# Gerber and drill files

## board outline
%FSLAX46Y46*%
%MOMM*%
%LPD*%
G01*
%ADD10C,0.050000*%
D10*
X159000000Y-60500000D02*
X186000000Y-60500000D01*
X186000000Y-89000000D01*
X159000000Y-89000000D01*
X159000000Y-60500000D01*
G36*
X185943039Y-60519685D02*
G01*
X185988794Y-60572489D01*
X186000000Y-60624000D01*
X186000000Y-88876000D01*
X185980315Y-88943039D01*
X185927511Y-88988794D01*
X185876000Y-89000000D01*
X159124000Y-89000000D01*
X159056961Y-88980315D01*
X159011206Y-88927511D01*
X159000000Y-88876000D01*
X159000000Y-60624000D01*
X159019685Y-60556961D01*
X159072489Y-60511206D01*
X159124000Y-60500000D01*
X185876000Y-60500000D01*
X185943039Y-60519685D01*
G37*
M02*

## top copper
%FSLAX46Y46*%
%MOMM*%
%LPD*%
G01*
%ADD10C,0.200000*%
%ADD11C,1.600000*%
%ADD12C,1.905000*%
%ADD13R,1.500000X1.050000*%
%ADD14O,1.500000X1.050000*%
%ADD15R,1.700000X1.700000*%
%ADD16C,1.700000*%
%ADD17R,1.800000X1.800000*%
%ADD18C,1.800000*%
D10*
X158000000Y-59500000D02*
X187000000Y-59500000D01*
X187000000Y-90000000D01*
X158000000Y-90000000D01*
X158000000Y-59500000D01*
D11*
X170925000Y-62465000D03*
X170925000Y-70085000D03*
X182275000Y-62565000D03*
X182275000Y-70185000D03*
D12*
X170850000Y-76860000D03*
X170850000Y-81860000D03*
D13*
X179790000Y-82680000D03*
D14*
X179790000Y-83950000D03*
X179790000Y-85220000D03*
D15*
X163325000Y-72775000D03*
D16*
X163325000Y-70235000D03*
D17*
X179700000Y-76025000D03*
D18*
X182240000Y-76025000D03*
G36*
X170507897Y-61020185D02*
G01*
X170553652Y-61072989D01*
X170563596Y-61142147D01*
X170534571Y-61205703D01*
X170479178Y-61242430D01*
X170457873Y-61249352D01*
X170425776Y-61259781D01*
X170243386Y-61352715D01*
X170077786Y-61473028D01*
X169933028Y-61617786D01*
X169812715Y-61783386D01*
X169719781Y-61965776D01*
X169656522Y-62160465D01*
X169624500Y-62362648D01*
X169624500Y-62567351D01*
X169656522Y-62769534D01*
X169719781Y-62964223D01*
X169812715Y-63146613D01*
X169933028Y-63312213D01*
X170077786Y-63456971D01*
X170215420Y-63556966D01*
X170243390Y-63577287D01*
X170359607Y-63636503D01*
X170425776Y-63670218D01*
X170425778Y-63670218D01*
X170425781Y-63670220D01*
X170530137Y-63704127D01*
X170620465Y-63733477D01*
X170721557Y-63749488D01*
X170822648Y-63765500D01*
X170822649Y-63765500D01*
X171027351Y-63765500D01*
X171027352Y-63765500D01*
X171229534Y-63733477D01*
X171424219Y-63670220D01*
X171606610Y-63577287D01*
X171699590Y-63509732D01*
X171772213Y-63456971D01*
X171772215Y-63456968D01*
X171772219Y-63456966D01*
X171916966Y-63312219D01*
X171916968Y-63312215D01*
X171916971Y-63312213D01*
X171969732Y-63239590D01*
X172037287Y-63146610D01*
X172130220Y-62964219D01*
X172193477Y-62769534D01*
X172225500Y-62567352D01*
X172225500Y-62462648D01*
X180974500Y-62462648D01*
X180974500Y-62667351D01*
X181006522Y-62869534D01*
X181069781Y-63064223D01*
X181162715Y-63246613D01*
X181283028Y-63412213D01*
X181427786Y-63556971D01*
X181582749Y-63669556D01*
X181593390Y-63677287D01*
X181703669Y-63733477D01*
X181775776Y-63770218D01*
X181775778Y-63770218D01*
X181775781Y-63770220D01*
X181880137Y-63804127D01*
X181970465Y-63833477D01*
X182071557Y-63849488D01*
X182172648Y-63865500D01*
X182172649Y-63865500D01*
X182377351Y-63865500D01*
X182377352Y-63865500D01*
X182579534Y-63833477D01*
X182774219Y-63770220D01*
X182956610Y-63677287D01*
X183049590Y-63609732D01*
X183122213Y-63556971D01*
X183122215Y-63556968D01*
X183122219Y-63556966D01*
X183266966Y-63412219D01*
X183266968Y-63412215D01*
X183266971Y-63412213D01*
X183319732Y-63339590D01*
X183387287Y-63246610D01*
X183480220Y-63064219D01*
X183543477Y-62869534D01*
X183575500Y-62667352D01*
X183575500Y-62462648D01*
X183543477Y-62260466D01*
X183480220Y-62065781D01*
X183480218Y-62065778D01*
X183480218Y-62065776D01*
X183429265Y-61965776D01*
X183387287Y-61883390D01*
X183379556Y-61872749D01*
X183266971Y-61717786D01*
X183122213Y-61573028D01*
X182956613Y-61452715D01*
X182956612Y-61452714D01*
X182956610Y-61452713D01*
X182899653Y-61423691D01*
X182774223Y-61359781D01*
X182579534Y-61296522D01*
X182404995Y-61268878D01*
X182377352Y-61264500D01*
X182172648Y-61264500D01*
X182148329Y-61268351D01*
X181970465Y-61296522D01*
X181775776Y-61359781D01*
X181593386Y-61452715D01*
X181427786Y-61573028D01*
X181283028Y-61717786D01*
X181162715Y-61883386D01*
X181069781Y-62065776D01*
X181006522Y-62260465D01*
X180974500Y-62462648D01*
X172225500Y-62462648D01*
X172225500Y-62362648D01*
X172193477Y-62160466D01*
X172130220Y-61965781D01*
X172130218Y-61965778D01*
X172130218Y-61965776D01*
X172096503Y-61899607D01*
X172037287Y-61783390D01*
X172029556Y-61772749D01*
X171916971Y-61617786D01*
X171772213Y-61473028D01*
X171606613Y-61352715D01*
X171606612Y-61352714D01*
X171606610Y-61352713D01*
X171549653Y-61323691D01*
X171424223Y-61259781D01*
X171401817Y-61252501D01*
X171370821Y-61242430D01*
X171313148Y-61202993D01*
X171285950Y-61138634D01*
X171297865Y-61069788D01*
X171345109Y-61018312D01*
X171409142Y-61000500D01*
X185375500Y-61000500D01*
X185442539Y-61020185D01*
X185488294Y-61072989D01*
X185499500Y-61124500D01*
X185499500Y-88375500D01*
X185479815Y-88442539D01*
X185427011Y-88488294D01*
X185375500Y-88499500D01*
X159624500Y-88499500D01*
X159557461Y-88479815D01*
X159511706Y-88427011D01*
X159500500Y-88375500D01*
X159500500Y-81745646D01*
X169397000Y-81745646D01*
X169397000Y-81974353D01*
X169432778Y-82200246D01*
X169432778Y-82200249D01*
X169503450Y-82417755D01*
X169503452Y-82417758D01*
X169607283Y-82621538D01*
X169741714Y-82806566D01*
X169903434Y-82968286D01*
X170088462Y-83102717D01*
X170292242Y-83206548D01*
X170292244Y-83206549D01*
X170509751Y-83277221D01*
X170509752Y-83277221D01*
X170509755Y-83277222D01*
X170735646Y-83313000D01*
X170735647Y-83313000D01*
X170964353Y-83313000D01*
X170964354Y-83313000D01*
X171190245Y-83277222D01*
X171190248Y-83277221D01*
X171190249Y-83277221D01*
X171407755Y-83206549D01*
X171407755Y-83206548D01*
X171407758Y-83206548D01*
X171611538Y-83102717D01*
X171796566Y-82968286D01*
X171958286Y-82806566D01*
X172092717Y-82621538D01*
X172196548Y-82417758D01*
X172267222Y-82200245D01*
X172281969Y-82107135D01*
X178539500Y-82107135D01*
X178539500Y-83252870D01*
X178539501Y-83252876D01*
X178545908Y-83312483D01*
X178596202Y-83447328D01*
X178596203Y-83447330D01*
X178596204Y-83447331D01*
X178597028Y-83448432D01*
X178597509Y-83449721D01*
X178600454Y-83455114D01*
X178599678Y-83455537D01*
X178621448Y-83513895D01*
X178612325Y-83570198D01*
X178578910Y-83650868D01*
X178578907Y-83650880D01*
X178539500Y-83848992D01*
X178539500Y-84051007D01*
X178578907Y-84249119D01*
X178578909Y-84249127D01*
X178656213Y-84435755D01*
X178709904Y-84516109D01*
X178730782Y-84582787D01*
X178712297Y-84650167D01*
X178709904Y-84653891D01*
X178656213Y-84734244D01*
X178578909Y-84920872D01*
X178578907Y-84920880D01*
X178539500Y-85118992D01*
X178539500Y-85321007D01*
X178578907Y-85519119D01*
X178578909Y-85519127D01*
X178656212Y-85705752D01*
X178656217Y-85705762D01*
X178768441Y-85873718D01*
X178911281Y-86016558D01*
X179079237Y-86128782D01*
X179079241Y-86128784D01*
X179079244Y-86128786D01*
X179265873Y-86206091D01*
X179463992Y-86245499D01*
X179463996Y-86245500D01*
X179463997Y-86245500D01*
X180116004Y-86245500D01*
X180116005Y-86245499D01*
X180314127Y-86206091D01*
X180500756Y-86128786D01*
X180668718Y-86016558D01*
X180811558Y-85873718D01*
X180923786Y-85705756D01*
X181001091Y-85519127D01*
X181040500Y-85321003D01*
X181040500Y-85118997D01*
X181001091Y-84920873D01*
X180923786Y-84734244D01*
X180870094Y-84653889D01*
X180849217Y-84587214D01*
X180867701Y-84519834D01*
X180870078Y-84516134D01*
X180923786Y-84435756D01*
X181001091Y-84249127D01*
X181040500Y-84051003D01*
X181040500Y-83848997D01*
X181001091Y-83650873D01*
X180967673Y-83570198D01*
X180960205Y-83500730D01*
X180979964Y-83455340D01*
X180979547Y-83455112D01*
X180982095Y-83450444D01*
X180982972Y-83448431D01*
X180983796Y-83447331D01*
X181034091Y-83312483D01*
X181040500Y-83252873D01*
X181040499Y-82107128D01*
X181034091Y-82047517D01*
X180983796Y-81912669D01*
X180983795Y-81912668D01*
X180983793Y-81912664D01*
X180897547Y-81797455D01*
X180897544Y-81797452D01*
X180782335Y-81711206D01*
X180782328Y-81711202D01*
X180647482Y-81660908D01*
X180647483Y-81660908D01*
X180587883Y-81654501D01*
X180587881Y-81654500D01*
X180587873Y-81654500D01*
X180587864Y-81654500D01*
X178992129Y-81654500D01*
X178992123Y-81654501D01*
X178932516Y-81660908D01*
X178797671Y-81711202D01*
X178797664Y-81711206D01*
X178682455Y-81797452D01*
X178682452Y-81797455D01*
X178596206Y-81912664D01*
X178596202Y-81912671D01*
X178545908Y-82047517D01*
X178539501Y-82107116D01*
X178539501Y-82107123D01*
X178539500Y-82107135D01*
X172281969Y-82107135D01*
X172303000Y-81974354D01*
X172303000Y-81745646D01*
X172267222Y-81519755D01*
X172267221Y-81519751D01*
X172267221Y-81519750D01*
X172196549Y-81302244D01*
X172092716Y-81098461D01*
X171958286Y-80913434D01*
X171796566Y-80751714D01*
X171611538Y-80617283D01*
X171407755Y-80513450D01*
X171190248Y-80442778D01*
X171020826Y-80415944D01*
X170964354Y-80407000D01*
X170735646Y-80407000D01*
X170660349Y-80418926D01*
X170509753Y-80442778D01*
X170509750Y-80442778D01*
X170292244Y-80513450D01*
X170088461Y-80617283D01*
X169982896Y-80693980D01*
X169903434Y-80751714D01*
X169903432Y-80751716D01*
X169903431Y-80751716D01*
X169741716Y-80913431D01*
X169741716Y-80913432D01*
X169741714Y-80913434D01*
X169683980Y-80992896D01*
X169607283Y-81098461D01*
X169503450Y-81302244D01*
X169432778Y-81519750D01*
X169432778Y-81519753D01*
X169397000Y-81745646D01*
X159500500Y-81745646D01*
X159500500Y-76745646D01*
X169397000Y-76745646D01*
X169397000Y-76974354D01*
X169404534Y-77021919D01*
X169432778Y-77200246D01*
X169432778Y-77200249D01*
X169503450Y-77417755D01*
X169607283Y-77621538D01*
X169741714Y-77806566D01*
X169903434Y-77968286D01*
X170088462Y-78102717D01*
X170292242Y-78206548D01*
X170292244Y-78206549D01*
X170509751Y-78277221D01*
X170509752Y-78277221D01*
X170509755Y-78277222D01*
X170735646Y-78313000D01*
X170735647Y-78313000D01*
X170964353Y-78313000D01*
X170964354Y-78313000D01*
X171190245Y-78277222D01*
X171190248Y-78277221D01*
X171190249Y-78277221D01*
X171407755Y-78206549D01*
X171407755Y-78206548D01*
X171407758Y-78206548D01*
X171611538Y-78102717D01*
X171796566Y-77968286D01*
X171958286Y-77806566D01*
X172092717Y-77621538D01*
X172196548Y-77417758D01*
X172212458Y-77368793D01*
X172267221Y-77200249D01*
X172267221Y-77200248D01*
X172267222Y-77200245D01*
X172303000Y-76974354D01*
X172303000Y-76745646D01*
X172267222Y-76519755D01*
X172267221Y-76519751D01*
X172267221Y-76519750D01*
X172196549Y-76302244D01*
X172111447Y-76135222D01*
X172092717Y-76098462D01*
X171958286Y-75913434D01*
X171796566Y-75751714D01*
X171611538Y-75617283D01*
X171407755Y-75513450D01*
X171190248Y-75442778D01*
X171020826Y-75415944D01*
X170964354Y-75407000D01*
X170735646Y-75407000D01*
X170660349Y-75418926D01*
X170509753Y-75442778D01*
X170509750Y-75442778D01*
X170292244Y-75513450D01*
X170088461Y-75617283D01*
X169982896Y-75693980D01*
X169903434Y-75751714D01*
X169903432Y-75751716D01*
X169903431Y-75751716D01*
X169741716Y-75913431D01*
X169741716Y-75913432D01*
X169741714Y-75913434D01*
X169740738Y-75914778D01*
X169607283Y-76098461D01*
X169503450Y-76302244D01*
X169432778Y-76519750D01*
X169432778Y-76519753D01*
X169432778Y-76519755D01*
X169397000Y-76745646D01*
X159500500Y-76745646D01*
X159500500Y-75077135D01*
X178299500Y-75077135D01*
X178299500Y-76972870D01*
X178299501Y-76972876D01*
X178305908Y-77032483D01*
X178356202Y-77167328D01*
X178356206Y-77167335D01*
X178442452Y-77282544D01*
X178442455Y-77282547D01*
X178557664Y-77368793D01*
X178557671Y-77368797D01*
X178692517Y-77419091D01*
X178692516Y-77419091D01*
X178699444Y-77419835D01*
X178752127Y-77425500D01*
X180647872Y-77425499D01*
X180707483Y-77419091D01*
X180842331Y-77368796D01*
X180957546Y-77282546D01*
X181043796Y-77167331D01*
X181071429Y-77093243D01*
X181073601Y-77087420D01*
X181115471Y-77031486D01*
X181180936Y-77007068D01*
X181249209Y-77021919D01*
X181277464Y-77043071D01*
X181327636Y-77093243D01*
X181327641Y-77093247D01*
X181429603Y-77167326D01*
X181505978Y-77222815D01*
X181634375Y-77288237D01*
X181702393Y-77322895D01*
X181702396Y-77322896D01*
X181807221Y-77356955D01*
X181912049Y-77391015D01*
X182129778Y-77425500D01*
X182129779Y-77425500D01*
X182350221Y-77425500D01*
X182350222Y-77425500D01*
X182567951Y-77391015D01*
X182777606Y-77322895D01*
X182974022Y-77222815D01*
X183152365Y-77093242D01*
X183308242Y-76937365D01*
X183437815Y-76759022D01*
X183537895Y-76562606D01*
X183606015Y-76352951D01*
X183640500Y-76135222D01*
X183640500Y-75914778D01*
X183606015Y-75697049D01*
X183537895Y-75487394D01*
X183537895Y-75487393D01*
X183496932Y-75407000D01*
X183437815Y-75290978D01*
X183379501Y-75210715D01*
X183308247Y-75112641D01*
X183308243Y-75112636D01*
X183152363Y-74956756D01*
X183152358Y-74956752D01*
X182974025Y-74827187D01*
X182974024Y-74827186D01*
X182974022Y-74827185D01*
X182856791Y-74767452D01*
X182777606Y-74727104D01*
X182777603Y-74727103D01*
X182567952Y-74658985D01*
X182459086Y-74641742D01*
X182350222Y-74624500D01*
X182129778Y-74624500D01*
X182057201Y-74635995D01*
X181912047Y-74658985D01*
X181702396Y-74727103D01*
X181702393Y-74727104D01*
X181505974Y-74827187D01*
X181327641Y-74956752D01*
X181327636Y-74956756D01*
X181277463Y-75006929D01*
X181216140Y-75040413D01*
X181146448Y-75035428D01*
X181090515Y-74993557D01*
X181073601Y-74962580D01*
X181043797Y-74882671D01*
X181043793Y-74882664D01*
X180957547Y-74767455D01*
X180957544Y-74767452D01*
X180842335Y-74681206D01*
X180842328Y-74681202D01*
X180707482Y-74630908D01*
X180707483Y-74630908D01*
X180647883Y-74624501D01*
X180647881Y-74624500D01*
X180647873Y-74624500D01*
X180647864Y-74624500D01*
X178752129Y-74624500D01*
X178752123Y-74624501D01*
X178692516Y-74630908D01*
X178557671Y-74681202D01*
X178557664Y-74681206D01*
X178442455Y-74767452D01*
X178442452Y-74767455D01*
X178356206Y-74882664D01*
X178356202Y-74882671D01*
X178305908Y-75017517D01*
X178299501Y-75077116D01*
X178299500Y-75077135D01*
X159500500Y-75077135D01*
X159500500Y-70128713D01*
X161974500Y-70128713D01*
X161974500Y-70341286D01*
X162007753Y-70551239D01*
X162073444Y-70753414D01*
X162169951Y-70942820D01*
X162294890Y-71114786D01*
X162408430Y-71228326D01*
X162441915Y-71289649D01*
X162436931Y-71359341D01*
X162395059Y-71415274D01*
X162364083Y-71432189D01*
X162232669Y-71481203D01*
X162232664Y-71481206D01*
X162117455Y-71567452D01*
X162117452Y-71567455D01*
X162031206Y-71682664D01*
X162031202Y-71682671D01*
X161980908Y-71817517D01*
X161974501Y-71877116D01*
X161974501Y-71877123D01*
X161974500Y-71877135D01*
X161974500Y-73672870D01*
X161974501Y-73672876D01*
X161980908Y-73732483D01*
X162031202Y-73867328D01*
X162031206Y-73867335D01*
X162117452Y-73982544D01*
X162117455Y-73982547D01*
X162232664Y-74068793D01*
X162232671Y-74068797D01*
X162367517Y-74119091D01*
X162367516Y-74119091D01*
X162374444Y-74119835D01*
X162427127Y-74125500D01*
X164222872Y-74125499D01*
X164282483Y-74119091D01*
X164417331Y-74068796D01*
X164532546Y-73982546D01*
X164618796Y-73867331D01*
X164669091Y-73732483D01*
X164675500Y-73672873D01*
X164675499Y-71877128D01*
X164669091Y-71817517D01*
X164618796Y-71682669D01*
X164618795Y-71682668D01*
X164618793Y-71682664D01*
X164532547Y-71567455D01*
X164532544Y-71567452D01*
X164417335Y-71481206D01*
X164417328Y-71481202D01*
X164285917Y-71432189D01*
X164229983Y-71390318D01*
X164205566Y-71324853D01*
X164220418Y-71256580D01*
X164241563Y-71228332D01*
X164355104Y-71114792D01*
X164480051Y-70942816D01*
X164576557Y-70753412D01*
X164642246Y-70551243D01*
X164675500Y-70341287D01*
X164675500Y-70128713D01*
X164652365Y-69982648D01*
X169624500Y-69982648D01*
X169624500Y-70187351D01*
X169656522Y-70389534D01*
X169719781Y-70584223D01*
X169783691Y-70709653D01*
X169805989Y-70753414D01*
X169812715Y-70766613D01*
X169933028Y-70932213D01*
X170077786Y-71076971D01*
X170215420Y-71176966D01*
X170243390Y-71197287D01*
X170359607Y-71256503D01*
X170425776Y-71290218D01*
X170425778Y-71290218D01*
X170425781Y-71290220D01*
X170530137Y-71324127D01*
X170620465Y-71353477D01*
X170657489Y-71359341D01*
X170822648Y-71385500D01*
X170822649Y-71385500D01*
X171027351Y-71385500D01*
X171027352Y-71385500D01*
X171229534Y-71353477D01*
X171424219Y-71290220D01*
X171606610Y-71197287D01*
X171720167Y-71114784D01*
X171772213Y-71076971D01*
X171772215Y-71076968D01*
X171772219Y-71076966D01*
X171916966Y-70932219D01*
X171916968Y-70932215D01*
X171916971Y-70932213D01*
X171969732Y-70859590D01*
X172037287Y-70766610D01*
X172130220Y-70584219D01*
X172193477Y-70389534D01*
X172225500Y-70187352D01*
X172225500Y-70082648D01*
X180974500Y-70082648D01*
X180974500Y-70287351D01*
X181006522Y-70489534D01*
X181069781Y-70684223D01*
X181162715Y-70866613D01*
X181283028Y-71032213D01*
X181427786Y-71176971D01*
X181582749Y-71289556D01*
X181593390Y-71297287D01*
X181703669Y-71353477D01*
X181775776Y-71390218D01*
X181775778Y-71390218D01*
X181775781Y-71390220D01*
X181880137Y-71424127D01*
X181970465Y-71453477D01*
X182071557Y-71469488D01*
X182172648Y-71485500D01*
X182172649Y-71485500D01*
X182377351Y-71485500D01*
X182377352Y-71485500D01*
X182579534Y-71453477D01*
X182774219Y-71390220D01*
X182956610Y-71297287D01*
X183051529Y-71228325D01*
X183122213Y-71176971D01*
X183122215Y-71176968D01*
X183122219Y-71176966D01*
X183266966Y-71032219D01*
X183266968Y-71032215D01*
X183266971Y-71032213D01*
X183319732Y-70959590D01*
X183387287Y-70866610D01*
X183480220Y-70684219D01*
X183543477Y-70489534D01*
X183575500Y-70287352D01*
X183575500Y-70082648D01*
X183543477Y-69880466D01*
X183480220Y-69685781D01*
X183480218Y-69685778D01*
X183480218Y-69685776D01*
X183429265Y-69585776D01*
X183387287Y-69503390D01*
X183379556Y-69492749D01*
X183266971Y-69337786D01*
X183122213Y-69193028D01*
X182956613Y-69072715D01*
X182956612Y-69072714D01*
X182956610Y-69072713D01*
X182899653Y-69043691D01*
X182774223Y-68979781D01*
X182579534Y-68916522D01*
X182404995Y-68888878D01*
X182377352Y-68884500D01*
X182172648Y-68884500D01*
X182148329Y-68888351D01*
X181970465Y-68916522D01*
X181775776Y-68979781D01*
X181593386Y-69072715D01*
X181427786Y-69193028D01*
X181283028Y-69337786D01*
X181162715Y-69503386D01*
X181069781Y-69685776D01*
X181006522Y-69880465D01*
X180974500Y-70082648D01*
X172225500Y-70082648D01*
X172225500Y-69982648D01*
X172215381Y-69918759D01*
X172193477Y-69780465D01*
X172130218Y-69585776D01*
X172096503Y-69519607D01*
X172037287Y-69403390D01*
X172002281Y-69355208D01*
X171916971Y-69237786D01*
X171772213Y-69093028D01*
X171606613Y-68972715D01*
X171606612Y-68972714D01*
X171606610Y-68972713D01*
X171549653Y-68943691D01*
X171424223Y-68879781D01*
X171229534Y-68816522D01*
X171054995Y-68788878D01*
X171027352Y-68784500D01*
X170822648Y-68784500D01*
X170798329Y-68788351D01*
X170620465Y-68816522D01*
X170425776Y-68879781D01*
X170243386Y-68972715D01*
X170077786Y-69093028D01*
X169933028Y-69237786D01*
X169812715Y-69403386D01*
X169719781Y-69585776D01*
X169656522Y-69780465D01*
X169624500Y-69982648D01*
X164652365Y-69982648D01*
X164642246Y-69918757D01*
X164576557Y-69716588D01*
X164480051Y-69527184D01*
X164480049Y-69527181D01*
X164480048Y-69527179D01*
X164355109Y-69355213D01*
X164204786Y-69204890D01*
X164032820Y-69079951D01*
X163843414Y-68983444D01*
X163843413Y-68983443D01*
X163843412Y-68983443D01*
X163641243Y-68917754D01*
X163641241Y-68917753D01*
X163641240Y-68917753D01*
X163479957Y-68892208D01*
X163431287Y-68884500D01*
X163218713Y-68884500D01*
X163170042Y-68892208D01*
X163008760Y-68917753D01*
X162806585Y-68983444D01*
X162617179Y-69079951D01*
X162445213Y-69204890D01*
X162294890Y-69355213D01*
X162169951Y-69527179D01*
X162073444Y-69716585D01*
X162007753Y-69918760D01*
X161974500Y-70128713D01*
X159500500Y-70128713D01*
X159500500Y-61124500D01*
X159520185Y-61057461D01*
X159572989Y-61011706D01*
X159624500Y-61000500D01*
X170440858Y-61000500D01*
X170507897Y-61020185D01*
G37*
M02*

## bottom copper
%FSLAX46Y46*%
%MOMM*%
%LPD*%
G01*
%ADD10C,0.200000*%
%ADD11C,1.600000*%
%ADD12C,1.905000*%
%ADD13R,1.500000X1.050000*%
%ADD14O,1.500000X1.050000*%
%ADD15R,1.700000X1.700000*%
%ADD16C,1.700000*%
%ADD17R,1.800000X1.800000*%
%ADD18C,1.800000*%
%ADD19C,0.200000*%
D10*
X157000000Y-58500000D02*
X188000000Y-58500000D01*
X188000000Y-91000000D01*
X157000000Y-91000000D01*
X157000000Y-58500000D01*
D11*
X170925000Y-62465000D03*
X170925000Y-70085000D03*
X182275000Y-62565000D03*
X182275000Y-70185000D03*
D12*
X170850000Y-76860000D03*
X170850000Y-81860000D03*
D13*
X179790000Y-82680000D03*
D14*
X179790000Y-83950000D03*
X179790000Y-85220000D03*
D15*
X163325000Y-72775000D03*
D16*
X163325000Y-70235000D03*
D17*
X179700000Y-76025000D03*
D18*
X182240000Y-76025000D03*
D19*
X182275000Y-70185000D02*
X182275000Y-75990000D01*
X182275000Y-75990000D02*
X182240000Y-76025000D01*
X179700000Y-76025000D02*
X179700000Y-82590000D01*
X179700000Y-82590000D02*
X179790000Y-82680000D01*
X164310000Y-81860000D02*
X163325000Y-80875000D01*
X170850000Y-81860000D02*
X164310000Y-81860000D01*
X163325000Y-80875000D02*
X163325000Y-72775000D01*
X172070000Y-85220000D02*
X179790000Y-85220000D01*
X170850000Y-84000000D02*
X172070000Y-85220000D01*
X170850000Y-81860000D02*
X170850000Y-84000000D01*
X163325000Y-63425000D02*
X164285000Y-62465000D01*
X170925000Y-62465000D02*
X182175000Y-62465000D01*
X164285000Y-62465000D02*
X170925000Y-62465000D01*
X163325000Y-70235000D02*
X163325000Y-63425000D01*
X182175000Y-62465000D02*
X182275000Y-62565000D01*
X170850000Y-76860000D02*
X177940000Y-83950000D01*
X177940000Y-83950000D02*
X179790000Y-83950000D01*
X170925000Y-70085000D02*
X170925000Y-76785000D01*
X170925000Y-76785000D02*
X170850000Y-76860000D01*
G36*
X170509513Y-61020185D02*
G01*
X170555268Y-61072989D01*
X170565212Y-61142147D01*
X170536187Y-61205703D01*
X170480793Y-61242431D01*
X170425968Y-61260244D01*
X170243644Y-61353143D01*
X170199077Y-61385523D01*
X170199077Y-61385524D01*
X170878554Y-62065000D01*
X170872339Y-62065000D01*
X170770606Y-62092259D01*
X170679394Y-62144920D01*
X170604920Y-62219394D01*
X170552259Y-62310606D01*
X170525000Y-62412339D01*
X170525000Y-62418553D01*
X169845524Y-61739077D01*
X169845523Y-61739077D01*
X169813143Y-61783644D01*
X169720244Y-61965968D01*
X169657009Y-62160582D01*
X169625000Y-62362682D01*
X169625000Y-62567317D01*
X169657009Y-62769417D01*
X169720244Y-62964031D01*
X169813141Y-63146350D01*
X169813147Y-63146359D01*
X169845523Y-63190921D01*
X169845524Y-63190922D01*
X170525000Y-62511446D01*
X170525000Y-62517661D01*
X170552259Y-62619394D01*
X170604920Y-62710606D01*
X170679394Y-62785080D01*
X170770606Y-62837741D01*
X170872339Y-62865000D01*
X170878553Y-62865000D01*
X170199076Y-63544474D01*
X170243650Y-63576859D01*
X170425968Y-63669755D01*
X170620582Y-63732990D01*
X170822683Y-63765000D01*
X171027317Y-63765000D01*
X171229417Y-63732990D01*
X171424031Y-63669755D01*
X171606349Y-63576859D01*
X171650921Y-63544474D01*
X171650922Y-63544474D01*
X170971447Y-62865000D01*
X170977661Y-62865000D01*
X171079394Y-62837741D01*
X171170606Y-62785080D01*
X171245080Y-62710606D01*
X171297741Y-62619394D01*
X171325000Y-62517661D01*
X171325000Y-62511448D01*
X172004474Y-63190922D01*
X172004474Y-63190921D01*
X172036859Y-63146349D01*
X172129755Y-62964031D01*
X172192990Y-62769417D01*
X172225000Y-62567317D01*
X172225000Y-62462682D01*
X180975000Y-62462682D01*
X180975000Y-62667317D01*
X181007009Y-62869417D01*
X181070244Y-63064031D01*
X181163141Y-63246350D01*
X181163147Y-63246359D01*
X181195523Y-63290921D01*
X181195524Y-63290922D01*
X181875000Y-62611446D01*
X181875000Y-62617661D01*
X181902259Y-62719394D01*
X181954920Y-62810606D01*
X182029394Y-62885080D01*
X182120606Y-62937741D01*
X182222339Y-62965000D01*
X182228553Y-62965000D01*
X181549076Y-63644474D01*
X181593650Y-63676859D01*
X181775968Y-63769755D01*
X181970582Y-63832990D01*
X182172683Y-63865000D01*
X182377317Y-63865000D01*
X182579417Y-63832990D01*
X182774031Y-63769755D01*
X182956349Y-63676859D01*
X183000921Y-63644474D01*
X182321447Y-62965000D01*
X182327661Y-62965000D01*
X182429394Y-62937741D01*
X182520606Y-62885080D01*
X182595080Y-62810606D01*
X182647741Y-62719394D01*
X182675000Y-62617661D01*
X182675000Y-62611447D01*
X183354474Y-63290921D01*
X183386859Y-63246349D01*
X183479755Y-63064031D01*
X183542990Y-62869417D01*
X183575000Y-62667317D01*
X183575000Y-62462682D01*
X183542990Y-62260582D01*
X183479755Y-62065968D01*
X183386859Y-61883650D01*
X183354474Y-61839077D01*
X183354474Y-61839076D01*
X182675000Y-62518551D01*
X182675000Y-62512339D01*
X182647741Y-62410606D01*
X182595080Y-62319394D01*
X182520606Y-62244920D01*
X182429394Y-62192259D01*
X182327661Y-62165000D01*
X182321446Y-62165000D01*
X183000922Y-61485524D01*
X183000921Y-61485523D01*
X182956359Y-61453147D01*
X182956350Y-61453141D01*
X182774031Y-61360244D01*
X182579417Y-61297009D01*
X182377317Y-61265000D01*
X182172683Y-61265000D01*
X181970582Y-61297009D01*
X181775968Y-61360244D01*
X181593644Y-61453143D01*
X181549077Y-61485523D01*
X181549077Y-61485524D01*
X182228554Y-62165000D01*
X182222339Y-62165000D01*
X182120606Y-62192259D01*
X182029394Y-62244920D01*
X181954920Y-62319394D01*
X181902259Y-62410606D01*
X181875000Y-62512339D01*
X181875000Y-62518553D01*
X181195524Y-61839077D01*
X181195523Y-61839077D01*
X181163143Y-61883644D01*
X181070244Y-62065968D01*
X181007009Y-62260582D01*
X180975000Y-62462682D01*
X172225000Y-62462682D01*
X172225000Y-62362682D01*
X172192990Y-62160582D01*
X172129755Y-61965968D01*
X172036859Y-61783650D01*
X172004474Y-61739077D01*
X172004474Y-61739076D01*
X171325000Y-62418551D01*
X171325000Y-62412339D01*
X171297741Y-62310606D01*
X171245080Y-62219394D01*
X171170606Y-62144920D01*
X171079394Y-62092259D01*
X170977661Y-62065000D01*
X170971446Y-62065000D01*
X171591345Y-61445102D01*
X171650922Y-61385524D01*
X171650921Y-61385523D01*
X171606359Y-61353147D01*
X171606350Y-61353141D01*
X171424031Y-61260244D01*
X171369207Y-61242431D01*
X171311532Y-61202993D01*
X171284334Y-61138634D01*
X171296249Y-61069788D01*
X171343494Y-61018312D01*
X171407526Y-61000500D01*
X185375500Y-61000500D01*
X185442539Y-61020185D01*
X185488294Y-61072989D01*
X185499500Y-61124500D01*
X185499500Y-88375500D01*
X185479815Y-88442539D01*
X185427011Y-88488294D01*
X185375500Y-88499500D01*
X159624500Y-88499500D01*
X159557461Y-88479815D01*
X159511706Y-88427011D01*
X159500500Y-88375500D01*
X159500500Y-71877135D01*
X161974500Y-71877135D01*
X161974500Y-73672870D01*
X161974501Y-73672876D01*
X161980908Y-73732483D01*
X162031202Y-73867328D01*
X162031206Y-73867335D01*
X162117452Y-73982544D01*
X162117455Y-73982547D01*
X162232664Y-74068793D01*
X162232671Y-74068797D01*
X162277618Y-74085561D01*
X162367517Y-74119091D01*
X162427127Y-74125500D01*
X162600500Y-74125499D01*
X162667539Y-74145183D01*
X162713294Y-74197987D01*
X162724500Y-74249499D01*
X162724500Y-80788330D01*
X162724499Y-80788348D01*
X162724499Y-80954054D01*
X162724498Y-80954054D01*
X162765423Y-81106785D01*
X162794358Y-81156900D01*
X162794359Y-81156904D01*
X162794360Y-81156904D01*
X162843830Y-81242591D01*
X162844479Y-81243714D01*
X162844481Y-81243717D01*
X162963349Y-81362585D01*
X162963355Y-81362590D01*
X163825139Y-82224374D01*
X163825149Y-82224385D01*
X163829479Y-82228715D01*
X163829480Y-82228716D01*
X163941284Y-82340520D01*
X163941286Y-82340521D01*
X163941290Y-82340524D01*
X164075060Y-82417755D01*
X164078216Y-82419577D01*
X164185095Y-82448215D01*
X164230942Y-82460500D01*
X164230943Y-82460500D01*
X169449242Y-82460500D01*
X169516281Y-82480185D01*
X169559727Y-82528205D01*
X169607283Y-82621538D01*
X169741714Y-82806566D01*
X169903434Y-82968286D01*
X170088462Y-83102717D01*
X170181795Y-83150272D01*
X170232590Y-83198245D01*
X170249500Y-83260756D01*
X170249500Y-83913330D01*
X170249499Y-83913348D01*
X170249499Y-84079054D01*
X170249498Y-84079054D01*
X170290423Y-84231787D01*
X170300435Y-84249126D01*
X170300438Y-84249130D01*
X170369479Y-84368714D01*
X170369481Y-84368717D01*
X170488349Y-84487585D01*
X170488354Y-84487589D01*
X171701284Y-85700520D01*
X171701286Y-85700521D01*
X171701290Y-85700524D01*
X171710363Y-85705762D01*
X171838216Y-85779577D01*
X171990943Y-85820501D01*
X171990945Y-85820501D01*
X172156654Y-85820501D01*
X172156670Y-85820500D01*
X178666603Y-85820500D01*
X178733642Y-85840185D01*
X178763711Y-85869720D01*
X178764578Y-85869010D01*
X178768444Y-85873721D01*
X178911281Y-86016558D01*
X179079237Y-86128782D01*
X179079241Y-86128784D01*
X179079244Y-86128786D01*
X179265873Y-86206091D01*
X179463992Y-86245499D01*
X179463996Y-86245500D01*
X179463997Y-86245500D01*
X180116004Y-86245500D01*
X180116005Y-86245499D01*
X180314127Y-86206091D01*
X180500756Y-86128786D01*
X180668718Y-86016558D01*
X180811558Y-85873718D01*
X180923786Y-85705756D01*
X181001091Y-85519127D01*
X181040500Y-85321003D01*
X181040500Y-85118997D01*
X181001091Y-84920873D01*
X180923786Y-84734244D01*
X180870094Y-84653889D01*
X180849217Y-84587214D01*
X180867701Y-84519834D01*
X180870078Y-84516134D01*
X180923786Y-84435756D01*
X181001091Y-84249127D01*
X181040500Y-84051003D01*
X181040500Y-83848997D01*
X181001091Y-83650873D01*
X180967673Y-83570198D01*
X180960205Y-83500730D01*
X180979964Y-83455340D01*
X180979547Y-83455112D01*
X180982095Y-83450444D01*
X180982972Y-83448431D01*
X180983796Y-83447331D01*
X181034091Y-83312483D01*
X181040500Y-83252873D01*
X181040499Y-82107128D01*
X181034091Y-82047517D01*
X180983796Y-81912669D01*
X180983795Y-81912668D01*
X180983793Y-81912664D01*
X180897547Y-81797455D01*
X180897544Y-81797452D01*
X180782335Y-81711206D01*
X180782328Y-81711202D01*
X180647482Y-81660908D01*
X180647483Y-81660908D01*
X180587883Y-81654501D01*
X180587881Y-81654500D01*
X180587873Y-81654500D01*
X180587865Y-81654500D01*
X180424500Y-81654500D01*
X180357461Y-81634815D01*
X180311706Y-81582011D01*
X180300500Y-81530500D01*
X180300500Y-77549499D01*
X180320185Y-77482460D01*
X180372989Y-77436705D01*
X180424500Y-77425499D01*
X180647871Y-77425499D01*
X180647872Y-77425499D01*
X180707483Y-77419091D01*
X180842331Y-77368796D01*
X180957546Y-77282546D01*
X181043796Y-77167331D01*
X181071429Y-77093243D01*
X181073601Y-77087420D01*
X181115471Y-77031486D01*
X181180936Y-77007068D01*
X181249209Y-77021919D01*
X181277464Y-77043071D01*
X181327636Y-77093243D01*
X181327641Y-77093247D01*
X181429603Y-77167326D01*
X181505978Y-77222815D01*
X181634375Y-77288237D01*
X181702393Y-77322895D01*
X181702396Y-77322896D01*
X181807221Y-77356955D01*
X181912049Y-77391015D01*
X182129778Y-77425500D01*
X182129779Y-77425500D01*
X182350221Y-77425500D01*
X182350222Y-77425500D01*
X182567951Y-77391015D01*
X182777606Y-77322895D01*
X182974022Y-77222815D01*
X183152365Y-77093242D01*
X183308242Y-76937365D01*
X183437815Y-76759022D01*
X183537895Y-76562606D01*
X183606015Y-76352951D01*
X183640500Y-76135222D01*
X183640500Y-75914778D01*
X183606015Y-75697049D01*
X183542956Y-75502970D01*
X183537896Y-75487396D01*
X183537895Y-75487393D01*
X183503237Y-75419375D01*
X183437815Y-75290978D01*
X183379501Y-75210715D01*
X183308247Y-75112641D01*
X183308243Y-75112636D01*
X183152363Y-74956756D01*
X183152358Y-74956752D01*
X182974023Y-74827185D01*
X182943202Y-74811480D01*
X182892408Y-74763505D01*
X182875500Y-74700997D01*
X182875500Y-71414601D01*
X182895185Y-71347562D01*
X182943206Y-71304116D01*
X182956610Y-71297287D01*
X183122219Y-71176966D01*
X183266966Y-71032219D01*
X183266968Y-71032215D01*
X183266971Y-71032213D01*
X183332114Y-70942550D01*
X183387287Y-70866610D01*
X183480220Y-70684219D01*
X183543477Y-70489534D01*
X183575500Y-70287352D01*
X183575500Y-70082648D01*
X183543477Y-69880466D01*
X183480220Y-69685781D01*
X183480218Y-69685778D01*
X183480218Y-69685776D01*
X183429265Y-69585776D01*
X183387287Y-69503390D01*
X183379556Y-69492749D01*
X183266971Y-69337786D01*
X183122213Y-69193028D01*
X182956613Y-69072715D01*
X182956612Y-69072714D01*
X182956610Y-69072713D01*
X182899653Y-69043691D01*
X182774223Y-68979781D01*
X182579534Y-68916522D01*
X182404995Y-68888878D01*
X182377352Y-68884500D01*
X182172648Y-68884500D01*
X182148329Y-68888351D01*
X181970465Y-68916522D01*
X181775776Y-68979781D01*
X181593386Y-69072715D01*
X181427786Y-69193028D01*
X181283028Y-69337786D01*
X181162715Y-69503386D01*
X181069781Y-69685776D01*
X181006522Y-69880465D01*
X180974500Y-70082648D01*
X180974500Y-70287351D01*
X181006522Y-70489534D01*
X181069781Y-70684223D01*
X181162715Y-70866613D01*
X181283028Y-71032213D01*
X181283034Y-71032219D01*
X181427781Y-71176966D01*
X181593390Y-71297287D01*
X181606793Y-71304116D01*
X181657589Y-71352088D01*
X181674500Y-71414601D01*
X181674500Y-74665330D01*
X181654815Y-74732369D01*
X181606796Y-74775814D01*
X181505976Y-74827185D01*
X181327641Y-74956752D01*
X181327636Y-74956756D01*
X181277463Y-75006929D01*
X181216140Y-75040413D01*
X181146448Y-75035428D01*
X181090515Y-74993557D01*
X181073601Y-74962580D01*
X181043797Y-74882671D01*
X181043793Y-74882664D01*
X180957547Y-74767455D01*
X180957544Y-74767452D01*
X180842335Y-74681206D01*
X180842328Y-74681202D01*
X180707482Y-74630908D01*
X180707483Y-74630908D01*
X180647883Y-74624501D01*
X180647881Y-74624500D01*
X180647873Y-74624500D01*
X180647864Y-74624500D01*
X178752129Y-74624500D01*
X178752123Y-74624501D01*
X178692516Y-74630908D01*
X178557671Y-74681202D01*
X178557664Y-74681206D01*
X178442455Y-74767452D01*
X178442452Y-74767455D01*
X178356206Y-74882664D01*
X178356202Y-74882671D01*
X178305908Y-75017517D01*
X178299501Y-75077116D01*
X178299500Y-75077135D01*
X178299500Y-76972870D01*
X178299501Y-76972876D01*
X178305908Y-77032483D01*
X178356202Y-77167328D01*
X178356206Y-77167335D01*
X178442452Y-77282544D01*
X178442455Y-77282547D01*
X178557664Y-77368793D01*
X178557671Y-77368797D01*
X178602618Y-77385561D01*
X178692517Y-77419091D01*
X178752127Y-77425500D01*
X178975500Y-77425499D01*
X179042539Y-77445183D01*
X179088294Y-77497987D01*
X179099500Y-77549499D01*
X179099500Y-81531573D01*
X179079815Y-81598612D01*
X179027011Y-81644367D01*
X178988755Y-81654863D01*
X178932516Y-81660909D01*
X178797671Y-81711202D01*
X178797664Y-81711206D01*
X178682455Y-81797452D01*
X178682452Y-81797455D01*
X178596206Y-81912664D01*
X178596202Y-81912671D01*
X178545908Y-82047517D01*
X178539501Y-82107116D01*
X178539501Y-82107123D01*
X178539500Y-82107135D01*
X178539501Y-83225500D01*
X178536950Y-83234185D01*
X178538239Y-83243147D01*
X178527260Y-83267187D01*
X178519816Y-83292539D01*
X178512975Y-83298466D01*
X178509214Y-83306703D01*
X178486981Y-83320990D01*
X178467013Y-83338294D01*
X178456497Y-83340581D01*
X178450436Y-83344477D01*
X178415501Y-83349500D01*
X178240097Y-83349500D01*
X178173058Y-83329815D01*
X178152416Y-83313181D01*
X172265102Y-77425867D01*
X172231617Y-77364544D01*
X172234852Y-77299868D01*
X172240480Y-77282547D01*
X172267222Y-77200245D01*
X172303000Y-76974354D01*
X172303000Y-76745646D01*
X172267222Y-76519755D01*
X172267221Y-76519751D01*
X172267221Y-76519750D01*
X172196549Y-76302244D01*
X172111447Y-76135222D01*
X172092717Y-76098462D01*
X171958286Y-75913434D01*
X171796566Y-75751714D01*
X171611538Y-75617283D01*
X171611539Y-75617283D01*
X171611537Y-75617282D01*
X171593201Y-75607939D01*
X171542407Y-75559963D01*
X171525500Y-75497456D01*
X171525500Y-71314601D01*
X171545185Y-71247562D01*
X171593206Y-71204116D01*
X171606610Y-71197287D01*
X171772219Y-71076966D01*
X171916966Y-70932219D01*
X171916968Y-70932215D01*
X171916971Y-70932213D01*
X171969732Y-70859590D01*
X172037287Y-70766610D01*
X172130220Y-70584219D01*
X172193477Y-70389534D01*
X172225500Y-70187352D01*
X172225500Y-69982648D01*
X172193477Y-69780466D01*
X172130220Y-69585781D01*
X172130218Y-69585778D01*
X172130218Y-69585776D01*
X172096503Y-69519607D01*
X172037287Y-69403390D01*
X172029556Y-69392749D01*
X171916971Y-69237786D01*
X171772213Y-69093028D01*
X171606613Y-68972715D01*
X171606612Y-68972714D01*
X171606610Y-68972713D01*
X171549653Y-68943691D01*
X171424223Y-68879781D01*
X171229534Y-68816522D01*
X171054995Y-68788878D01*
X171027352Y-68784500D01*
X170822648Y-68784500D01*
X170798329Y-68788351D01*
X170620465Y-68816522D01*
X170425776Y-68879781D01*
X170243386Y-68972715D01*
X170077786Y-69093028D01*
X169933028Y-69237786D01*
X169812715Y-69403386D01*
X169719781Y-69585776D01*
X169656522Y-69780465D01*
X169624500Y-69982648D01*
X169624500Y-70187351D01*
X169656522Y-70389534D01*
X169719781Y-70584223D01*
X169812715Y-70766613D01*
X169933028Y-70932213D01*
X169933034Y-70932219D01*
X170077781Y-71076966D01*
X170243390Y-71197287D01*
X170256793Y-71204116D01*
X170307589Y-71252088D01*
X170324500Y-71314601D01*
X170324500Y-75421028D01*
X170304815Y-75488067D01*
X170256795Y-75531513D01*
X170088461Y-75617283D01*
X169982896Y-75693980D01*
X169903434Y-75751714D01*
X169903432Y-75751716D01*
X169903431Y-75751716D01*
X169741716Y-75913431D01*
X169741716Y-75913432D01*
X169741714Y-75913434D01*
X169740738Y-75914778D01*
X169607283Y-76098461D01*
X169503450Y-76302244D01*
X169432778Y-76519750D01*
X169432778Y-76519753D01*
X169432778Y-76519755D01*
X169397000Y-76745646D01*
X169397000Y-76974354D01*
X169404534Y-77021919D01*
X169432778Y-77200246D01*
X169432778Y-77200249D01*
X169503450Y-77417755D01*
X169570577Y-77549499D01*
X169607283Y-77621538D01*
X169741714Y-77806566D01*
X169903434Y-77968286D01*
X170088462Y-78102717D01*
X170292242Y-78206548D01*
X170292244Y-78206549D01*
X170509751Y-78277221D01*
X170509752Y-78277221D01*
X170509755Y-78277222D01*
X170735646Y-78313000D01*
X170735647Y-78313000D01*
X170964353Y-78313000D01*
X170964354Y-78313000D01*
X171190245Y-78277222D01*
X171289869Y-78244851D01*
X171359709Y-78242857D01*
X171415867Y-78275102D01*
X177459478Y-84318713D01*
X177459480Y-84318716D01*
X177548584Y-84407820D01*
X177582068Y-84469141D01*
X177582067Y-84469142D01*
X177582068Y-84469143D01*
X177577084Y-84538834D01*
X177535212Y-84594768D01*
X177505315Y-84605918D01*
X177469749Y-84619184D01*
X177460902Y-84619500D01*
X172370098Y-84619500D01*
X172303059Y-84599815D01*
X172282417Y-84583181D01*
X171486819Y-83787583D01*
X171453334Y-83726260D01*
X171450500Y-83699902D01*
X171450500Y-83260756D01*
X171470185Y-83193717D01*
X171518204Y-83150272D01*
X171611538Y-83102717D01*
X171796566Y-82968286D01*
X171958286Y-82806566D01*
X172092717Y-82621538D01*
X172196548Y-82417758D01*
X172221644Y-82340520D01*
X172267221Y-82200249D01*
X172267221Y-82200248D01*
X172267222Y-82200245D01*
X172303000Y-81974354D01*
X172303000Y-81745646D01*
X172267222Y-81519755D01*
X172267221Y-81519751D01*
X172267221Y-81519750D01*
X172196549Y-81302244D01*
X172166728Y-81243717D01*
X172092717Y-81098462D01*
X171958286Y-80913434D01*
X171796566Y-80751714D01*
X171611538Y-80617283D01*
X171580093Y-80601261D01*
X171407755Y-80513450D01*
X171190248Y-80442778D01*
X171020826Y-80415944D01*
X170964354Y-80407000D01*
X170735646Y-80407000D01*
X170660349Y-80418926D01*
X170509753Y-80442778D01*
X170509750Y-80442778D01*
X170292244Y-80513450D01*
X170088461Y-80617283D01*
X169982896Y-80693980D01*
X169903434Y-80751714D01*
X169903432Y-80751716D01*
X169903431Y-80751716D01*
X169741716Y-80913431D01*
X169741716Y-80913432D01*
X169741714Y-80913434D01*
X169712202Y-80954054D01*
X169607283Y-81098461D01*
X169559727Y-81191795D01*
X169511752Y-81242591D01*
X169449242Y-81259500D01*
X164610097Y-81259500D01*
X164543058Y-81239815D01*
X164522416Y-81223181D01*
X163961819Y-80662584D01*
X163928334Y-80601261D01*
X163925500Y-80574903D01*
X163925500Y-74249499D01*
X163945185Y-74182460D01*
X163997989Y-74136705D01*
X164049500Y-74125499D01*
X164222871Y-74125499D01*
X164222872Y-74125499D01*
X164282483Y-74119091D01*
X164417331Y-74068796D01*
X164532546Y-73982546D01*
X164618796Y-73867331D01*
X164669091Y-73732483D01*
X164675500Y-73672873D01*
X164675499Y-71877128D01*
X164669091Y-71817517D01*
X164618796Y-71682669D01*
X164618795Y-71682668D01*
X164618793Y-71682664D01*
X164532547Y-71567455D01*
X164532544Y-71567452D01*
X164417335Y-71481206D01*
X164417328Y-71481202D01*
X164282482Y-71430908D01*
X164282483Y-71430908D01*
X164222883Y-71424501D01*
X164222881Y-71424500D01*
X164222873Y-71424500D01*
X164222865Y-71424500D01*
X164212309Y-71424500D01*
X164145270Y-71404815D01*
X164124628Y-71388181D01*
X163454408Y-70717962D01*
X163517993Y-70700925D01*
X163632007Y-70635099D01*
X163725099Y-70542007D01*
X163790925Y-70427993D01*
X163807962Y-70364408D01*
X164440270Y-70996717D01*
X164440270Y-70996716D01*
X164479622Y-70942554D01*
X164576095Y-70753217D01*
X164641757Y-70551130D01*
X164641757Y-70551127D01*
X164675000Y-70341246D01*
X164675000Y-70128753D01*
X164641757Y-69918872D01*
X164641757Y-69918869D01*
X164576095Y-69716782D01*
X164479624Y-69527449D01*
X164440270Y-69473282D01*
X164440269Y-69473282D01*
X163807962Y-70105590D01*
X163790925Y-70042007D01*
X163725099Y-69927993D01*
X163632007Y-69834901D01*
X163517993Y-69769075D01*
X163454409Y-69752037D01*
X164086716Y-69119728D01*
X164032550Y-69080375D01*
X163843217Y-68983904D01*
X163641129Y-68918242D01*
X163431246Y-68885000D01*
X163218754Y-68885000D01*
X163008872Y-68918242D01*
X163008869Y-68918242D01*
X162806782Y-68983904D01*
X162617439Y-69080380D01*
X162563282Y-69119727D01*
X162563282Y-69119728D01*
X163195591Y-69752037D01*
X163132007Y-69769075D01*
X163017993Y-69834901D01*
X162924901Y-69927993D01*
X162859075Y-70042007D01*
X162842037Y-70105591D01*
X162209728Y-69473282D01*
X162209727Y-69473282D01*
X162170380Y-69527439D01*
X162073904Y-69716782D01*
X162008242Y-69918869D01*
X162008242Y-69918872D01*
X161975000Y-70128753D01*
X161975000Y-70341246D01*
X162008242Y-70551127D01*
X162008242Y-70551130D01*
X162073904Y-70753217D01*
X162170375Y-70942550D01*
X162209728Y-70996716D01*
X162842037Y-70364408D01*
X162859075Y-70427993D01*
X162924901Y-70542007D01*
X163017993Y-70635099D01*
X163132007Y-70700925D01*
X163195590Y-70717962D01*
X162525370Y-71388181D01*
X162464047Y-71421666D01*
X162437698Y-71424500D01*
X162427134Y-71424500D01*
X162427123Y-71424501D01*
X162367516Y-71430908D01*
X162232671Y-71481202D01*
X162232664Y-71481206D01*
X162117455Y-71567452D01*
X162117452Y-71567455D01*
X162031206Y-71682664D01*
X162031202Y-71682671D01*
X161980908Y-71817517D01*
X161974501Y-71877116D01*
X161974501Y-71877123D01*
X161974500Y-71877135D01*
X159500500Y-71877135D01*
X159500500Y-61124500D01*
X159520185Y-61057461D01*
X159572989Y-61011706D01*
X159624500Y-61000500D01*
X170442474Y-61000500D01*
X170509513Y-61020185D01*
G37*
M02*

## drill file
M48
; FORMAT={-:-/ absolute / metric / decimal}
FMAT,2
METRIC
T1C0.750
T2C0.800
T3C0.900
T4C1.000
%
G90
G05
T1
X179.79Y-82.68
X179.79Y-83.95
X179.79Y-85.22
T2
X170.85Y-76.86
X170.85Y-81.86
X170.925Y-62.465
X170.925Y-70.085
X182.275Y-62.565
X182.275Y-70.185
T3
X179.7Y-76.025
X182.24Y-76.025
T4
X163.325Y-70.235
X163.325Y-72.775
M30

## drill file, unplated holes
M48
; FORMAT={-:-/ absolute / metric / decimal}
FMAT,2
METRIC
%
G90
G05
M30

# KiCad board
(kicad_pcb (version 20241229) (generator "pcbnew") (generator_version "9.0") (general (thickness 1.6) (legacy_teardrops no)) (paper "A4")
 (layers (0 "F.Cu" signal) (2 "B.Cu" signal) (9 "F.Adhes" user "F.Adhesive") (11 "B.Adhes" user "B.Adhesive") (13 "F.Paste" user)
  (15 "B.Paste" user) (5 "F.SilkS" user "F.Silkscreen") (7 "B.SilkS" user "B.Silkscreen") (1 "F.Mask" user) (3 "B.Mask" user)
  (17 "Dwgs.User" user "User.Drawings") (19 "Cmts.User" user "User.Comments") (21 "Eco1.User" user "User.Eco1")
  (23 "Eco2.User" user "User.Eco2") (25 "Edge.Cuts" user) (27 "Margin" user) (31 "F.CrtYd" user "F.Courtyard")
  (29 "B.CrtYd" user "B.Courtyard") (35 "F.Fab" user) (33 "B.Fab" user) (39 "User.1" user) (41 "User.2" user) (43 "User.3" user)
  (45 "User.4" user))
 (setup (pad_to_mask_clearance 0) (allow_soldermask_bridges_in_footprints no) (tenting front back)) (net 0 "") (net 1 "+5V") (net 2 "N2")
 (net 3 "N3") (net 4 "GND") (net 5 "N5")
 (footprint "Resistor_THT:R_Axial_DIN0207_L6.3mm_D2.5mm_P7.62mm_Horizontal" (layer "F.Cu") (at 170.925 62.465 -90)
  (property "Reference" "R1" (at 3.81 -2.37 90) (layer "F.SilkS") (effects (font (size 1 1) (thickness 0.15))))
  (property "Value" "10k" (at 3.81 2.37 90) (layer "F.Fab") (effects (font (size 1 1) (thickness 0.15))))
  (pad "1" thru_hole circle (at 0 0 270) (size 1.6 1.6) (drill 0.8) (layers "*.Cu" "*.Mask") (remove_unused_layers no) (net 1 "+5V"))
  (pad "2" thru_hole circle (at 7.62 0 270) (size 1.6 1.6) (drill 0.8) (layers "*.Cu" "*.Mask") (remove_unused_layers no) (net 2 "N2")))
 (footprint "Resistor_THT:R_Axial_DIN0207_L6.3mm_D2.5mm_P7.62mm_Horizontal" (layer "F.Cu") (at 182.275 62.565 -90)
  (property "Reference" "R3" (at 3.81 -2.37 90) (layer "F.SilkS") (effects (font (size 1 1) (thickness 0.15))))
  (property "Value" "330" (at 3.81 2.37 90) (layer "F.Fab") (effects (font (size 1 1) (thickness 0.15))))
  (pad "1" thru_hole circle (at 0 0 270) (size 1.6 1.6) (drill 0.8) (layers "*.Cu" "*.Mask") (remove_unused_layers no) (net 1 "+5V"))
  (pad "2" thru_hole circle (at 7.62 0 270) (size 1.6 1.6) (drill 0.8) (layers "*.Cu" "*.Mask") (remove_unused_layers no) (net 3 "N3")))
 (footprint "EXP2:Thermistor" (layer "F.Cu") (at 170.85 76.86 -90)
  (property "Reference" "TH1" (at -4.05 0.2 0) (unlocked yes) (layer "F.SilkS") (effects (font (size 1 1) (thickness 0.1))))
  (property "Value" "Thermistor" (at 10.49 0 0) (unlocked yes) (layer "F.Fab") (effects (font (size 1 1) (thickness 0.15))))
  (pad "1" thru_hole circle (at 0 0 270) (size 1.905 1.905) (drill 0.8) (layers "*.Cu" "*.Mask") (remove_unused_layers no) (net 2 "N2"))
  (pad "2" thru_hole circle (at 5 0 270) (size 1.905 1.905) (drill 0.8) (layers "*.Cu" "*.Mask") (remove_unused_layers no) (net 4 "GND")))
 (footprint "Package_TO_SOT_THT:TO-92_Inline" (layer "F.Cu") (at 179.79 82.68 -90)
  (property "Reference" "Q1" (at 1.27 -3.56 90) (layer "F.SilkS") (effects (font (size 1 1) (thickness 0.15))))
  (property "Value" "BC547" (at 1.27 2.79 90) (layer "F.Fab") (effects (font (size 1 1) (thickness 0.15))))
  (pad "1" thru_hole rect (at 0 0 270) (size 1.05 1.5) (drill 0.75) (layers "*.Cu" "*.Mask") (remove_unused_layers no) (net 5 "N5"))
  (pad "2" thru_hole oval (at 1.27 0 270) (size 1.05 1.5) (drill 0.75) (layers "*.Cu" "*.Mask") (remove_unused_layers no) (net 2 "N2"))
  (pad "3" thru_hole oval (at 2.54 0 270) (size 1.05 1.5) (drill 0.75) (layers "*.Cu" "*.Mask") (remove_unused_layers no) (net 4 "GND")))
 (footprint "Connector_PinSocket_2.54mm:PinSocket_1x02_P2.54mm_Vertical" (layer "F.Cu") (at 163.325 72.775 180)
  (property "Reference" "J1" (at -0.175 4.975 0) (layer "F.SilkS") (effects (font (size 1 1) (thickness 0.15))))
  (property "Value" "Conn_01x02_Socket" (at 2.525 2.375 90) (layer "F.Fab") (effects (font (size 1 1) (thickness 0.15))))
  (pad "1" thru_hole rect (at 0 0 180) (size 1.7 1.7) (drill 1) (layers "*.Cu" "*.Mask") (remove_unused_layers no) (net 4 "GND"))
  (pad "2" thru_hole circle (at 0 2.54 180) (size 1.7 1.7) (drill 1) (layers "*.Cu" "*.Mask") (remove_unused_layers no) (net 1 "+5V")))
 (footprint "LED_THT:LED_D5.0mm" (layer "F.Cu") (at 179.7 76.025)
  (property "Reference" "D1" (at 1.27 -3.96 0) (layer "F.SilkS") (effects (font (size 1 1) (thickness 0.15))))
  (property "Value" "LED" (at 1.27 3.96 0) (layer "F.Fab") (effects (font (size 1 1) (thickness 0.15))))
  (pad "1" thru_hole rect (at 0 0) (size 1.8 1.8) (drill 0.9) (layers "*.Cu" "*.Mask") (remove_unused_layers no) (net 5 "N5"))
  (pad "2" thru_hole circle (at 2.54 0) (size 1.8 1.8) (drill 0.9) (layers "*.Cu" "*.Mask") (remove_unused_layers no) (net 3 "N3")))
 (gr_rect (start 158 59.5) (end 187 90) (stroke (width 0.2) (type default)) (fill no) (layer "F.Cu"))
 (gr_rect (start 157 58.5) (end 188 91) (stroke (width 0.2) (type default)) (fill no) (layer "B.Cu"))
 (gr_rect (start 159 60.5) (end 186 89) (stroke (width 0.05) (type default)) (fill no) (layer "Edge.Cuts"))
 (segment (start 182.275 70.185) (end 182.275 75.99) (width 0.2) (layer "B.Cu") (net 3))
 (segment (start 182.275 75.99) (end 182.24 76.025) (width 0.2) (layer "B.Cu") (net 3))
 (segment (start 179.7 76.025) (end 179.7 82.59) (width 0.2) (layer "B.Cu") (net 5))
 (segment (start 179.7 82.59) (end 179.79 82.68) (width 0.2) (layer "B.Cu") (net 5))
 (segment (start 164.31 81.86) (end 163.325 80.875) (width 0.2) (layer "B.Cu") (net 4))
 (segment (start 170.85 81.86) (end 164.31 81.86) (width 0.2) (layer "B.Cu") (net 4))
 (segment (start 163.325 80.875) (end 163.325 72.775) (width 0.2) (layer "B.Cu") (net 4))
 (segment (start 172.07 85.22) (end 179.79 85.22) (width 0.2) (layer "B.Cu") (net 4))
 (segment (start 170.85 84) (end 172.07 85.22) (width 0.2) (layer "B.Cu") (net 4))
 (segment (start 170.85 81.86) (end 170.85 84) (width 0.2) (layer "B.Cu") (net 4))
 (segment (start 163.325 63.425) (end 164.285 62.465) (width 0.2) (layer "B.Cu") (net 1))
 (segment (start 170.925 62.465) (end 182.175 62.465) (width 0.2) (layer "B.Cu") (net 1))
 (segment (start 164.285 62.465) (end 170.925 62.465) (width 0.2) (layer "B.Cu") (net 1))
 (segment (start 163.325 70.235) (end 163.325 63.425) (width 0.2) (layer "B.Cu") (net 1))
 (segment (start 182.175 62.465) (end 182.275 62.565) (width 0.2) (layer "B.Cu") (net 1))
 (segment (start 170.85 76.86) (end 177.94 83.95) (width 0.2) (layer "B.Cu") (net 2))
 (segment (start 177.94 83.95) (end 179.79 83.95) (width 0.2) (layer "B.Cu") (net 2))
 (segment (start 170.925 70.085) (end 170.925 76.785) (width 0.2) (layer "B.Cu") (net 2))
 (segment (start 170.925 76.785) (end 170.85 76.86) (width 0.2) (layer "B.Cu") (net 2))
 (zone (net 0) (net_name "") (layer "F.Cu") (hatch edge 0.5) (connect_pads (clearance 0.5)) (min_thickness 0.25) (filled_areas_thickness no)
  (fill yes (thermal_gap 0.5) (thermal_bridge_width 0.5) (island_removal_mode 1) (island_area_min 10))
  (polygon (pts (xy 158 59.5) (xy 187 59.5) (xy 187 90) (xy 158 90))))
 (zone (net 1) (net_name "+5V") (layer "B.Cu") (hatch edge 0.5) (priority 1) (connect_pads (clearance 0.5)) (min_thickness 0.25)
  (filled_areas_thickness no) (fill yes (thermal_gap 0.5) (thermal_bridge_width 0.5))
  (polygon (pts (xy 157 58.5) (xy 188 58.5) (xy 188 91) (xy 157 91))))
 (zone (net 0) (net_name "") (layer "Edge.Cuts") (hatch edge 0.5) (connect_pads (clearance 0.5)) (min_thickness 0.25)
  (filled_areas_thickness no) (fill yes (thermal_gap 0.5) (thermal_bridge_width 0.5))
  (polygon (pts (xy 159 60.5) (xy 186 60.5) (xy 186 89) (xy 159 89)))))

